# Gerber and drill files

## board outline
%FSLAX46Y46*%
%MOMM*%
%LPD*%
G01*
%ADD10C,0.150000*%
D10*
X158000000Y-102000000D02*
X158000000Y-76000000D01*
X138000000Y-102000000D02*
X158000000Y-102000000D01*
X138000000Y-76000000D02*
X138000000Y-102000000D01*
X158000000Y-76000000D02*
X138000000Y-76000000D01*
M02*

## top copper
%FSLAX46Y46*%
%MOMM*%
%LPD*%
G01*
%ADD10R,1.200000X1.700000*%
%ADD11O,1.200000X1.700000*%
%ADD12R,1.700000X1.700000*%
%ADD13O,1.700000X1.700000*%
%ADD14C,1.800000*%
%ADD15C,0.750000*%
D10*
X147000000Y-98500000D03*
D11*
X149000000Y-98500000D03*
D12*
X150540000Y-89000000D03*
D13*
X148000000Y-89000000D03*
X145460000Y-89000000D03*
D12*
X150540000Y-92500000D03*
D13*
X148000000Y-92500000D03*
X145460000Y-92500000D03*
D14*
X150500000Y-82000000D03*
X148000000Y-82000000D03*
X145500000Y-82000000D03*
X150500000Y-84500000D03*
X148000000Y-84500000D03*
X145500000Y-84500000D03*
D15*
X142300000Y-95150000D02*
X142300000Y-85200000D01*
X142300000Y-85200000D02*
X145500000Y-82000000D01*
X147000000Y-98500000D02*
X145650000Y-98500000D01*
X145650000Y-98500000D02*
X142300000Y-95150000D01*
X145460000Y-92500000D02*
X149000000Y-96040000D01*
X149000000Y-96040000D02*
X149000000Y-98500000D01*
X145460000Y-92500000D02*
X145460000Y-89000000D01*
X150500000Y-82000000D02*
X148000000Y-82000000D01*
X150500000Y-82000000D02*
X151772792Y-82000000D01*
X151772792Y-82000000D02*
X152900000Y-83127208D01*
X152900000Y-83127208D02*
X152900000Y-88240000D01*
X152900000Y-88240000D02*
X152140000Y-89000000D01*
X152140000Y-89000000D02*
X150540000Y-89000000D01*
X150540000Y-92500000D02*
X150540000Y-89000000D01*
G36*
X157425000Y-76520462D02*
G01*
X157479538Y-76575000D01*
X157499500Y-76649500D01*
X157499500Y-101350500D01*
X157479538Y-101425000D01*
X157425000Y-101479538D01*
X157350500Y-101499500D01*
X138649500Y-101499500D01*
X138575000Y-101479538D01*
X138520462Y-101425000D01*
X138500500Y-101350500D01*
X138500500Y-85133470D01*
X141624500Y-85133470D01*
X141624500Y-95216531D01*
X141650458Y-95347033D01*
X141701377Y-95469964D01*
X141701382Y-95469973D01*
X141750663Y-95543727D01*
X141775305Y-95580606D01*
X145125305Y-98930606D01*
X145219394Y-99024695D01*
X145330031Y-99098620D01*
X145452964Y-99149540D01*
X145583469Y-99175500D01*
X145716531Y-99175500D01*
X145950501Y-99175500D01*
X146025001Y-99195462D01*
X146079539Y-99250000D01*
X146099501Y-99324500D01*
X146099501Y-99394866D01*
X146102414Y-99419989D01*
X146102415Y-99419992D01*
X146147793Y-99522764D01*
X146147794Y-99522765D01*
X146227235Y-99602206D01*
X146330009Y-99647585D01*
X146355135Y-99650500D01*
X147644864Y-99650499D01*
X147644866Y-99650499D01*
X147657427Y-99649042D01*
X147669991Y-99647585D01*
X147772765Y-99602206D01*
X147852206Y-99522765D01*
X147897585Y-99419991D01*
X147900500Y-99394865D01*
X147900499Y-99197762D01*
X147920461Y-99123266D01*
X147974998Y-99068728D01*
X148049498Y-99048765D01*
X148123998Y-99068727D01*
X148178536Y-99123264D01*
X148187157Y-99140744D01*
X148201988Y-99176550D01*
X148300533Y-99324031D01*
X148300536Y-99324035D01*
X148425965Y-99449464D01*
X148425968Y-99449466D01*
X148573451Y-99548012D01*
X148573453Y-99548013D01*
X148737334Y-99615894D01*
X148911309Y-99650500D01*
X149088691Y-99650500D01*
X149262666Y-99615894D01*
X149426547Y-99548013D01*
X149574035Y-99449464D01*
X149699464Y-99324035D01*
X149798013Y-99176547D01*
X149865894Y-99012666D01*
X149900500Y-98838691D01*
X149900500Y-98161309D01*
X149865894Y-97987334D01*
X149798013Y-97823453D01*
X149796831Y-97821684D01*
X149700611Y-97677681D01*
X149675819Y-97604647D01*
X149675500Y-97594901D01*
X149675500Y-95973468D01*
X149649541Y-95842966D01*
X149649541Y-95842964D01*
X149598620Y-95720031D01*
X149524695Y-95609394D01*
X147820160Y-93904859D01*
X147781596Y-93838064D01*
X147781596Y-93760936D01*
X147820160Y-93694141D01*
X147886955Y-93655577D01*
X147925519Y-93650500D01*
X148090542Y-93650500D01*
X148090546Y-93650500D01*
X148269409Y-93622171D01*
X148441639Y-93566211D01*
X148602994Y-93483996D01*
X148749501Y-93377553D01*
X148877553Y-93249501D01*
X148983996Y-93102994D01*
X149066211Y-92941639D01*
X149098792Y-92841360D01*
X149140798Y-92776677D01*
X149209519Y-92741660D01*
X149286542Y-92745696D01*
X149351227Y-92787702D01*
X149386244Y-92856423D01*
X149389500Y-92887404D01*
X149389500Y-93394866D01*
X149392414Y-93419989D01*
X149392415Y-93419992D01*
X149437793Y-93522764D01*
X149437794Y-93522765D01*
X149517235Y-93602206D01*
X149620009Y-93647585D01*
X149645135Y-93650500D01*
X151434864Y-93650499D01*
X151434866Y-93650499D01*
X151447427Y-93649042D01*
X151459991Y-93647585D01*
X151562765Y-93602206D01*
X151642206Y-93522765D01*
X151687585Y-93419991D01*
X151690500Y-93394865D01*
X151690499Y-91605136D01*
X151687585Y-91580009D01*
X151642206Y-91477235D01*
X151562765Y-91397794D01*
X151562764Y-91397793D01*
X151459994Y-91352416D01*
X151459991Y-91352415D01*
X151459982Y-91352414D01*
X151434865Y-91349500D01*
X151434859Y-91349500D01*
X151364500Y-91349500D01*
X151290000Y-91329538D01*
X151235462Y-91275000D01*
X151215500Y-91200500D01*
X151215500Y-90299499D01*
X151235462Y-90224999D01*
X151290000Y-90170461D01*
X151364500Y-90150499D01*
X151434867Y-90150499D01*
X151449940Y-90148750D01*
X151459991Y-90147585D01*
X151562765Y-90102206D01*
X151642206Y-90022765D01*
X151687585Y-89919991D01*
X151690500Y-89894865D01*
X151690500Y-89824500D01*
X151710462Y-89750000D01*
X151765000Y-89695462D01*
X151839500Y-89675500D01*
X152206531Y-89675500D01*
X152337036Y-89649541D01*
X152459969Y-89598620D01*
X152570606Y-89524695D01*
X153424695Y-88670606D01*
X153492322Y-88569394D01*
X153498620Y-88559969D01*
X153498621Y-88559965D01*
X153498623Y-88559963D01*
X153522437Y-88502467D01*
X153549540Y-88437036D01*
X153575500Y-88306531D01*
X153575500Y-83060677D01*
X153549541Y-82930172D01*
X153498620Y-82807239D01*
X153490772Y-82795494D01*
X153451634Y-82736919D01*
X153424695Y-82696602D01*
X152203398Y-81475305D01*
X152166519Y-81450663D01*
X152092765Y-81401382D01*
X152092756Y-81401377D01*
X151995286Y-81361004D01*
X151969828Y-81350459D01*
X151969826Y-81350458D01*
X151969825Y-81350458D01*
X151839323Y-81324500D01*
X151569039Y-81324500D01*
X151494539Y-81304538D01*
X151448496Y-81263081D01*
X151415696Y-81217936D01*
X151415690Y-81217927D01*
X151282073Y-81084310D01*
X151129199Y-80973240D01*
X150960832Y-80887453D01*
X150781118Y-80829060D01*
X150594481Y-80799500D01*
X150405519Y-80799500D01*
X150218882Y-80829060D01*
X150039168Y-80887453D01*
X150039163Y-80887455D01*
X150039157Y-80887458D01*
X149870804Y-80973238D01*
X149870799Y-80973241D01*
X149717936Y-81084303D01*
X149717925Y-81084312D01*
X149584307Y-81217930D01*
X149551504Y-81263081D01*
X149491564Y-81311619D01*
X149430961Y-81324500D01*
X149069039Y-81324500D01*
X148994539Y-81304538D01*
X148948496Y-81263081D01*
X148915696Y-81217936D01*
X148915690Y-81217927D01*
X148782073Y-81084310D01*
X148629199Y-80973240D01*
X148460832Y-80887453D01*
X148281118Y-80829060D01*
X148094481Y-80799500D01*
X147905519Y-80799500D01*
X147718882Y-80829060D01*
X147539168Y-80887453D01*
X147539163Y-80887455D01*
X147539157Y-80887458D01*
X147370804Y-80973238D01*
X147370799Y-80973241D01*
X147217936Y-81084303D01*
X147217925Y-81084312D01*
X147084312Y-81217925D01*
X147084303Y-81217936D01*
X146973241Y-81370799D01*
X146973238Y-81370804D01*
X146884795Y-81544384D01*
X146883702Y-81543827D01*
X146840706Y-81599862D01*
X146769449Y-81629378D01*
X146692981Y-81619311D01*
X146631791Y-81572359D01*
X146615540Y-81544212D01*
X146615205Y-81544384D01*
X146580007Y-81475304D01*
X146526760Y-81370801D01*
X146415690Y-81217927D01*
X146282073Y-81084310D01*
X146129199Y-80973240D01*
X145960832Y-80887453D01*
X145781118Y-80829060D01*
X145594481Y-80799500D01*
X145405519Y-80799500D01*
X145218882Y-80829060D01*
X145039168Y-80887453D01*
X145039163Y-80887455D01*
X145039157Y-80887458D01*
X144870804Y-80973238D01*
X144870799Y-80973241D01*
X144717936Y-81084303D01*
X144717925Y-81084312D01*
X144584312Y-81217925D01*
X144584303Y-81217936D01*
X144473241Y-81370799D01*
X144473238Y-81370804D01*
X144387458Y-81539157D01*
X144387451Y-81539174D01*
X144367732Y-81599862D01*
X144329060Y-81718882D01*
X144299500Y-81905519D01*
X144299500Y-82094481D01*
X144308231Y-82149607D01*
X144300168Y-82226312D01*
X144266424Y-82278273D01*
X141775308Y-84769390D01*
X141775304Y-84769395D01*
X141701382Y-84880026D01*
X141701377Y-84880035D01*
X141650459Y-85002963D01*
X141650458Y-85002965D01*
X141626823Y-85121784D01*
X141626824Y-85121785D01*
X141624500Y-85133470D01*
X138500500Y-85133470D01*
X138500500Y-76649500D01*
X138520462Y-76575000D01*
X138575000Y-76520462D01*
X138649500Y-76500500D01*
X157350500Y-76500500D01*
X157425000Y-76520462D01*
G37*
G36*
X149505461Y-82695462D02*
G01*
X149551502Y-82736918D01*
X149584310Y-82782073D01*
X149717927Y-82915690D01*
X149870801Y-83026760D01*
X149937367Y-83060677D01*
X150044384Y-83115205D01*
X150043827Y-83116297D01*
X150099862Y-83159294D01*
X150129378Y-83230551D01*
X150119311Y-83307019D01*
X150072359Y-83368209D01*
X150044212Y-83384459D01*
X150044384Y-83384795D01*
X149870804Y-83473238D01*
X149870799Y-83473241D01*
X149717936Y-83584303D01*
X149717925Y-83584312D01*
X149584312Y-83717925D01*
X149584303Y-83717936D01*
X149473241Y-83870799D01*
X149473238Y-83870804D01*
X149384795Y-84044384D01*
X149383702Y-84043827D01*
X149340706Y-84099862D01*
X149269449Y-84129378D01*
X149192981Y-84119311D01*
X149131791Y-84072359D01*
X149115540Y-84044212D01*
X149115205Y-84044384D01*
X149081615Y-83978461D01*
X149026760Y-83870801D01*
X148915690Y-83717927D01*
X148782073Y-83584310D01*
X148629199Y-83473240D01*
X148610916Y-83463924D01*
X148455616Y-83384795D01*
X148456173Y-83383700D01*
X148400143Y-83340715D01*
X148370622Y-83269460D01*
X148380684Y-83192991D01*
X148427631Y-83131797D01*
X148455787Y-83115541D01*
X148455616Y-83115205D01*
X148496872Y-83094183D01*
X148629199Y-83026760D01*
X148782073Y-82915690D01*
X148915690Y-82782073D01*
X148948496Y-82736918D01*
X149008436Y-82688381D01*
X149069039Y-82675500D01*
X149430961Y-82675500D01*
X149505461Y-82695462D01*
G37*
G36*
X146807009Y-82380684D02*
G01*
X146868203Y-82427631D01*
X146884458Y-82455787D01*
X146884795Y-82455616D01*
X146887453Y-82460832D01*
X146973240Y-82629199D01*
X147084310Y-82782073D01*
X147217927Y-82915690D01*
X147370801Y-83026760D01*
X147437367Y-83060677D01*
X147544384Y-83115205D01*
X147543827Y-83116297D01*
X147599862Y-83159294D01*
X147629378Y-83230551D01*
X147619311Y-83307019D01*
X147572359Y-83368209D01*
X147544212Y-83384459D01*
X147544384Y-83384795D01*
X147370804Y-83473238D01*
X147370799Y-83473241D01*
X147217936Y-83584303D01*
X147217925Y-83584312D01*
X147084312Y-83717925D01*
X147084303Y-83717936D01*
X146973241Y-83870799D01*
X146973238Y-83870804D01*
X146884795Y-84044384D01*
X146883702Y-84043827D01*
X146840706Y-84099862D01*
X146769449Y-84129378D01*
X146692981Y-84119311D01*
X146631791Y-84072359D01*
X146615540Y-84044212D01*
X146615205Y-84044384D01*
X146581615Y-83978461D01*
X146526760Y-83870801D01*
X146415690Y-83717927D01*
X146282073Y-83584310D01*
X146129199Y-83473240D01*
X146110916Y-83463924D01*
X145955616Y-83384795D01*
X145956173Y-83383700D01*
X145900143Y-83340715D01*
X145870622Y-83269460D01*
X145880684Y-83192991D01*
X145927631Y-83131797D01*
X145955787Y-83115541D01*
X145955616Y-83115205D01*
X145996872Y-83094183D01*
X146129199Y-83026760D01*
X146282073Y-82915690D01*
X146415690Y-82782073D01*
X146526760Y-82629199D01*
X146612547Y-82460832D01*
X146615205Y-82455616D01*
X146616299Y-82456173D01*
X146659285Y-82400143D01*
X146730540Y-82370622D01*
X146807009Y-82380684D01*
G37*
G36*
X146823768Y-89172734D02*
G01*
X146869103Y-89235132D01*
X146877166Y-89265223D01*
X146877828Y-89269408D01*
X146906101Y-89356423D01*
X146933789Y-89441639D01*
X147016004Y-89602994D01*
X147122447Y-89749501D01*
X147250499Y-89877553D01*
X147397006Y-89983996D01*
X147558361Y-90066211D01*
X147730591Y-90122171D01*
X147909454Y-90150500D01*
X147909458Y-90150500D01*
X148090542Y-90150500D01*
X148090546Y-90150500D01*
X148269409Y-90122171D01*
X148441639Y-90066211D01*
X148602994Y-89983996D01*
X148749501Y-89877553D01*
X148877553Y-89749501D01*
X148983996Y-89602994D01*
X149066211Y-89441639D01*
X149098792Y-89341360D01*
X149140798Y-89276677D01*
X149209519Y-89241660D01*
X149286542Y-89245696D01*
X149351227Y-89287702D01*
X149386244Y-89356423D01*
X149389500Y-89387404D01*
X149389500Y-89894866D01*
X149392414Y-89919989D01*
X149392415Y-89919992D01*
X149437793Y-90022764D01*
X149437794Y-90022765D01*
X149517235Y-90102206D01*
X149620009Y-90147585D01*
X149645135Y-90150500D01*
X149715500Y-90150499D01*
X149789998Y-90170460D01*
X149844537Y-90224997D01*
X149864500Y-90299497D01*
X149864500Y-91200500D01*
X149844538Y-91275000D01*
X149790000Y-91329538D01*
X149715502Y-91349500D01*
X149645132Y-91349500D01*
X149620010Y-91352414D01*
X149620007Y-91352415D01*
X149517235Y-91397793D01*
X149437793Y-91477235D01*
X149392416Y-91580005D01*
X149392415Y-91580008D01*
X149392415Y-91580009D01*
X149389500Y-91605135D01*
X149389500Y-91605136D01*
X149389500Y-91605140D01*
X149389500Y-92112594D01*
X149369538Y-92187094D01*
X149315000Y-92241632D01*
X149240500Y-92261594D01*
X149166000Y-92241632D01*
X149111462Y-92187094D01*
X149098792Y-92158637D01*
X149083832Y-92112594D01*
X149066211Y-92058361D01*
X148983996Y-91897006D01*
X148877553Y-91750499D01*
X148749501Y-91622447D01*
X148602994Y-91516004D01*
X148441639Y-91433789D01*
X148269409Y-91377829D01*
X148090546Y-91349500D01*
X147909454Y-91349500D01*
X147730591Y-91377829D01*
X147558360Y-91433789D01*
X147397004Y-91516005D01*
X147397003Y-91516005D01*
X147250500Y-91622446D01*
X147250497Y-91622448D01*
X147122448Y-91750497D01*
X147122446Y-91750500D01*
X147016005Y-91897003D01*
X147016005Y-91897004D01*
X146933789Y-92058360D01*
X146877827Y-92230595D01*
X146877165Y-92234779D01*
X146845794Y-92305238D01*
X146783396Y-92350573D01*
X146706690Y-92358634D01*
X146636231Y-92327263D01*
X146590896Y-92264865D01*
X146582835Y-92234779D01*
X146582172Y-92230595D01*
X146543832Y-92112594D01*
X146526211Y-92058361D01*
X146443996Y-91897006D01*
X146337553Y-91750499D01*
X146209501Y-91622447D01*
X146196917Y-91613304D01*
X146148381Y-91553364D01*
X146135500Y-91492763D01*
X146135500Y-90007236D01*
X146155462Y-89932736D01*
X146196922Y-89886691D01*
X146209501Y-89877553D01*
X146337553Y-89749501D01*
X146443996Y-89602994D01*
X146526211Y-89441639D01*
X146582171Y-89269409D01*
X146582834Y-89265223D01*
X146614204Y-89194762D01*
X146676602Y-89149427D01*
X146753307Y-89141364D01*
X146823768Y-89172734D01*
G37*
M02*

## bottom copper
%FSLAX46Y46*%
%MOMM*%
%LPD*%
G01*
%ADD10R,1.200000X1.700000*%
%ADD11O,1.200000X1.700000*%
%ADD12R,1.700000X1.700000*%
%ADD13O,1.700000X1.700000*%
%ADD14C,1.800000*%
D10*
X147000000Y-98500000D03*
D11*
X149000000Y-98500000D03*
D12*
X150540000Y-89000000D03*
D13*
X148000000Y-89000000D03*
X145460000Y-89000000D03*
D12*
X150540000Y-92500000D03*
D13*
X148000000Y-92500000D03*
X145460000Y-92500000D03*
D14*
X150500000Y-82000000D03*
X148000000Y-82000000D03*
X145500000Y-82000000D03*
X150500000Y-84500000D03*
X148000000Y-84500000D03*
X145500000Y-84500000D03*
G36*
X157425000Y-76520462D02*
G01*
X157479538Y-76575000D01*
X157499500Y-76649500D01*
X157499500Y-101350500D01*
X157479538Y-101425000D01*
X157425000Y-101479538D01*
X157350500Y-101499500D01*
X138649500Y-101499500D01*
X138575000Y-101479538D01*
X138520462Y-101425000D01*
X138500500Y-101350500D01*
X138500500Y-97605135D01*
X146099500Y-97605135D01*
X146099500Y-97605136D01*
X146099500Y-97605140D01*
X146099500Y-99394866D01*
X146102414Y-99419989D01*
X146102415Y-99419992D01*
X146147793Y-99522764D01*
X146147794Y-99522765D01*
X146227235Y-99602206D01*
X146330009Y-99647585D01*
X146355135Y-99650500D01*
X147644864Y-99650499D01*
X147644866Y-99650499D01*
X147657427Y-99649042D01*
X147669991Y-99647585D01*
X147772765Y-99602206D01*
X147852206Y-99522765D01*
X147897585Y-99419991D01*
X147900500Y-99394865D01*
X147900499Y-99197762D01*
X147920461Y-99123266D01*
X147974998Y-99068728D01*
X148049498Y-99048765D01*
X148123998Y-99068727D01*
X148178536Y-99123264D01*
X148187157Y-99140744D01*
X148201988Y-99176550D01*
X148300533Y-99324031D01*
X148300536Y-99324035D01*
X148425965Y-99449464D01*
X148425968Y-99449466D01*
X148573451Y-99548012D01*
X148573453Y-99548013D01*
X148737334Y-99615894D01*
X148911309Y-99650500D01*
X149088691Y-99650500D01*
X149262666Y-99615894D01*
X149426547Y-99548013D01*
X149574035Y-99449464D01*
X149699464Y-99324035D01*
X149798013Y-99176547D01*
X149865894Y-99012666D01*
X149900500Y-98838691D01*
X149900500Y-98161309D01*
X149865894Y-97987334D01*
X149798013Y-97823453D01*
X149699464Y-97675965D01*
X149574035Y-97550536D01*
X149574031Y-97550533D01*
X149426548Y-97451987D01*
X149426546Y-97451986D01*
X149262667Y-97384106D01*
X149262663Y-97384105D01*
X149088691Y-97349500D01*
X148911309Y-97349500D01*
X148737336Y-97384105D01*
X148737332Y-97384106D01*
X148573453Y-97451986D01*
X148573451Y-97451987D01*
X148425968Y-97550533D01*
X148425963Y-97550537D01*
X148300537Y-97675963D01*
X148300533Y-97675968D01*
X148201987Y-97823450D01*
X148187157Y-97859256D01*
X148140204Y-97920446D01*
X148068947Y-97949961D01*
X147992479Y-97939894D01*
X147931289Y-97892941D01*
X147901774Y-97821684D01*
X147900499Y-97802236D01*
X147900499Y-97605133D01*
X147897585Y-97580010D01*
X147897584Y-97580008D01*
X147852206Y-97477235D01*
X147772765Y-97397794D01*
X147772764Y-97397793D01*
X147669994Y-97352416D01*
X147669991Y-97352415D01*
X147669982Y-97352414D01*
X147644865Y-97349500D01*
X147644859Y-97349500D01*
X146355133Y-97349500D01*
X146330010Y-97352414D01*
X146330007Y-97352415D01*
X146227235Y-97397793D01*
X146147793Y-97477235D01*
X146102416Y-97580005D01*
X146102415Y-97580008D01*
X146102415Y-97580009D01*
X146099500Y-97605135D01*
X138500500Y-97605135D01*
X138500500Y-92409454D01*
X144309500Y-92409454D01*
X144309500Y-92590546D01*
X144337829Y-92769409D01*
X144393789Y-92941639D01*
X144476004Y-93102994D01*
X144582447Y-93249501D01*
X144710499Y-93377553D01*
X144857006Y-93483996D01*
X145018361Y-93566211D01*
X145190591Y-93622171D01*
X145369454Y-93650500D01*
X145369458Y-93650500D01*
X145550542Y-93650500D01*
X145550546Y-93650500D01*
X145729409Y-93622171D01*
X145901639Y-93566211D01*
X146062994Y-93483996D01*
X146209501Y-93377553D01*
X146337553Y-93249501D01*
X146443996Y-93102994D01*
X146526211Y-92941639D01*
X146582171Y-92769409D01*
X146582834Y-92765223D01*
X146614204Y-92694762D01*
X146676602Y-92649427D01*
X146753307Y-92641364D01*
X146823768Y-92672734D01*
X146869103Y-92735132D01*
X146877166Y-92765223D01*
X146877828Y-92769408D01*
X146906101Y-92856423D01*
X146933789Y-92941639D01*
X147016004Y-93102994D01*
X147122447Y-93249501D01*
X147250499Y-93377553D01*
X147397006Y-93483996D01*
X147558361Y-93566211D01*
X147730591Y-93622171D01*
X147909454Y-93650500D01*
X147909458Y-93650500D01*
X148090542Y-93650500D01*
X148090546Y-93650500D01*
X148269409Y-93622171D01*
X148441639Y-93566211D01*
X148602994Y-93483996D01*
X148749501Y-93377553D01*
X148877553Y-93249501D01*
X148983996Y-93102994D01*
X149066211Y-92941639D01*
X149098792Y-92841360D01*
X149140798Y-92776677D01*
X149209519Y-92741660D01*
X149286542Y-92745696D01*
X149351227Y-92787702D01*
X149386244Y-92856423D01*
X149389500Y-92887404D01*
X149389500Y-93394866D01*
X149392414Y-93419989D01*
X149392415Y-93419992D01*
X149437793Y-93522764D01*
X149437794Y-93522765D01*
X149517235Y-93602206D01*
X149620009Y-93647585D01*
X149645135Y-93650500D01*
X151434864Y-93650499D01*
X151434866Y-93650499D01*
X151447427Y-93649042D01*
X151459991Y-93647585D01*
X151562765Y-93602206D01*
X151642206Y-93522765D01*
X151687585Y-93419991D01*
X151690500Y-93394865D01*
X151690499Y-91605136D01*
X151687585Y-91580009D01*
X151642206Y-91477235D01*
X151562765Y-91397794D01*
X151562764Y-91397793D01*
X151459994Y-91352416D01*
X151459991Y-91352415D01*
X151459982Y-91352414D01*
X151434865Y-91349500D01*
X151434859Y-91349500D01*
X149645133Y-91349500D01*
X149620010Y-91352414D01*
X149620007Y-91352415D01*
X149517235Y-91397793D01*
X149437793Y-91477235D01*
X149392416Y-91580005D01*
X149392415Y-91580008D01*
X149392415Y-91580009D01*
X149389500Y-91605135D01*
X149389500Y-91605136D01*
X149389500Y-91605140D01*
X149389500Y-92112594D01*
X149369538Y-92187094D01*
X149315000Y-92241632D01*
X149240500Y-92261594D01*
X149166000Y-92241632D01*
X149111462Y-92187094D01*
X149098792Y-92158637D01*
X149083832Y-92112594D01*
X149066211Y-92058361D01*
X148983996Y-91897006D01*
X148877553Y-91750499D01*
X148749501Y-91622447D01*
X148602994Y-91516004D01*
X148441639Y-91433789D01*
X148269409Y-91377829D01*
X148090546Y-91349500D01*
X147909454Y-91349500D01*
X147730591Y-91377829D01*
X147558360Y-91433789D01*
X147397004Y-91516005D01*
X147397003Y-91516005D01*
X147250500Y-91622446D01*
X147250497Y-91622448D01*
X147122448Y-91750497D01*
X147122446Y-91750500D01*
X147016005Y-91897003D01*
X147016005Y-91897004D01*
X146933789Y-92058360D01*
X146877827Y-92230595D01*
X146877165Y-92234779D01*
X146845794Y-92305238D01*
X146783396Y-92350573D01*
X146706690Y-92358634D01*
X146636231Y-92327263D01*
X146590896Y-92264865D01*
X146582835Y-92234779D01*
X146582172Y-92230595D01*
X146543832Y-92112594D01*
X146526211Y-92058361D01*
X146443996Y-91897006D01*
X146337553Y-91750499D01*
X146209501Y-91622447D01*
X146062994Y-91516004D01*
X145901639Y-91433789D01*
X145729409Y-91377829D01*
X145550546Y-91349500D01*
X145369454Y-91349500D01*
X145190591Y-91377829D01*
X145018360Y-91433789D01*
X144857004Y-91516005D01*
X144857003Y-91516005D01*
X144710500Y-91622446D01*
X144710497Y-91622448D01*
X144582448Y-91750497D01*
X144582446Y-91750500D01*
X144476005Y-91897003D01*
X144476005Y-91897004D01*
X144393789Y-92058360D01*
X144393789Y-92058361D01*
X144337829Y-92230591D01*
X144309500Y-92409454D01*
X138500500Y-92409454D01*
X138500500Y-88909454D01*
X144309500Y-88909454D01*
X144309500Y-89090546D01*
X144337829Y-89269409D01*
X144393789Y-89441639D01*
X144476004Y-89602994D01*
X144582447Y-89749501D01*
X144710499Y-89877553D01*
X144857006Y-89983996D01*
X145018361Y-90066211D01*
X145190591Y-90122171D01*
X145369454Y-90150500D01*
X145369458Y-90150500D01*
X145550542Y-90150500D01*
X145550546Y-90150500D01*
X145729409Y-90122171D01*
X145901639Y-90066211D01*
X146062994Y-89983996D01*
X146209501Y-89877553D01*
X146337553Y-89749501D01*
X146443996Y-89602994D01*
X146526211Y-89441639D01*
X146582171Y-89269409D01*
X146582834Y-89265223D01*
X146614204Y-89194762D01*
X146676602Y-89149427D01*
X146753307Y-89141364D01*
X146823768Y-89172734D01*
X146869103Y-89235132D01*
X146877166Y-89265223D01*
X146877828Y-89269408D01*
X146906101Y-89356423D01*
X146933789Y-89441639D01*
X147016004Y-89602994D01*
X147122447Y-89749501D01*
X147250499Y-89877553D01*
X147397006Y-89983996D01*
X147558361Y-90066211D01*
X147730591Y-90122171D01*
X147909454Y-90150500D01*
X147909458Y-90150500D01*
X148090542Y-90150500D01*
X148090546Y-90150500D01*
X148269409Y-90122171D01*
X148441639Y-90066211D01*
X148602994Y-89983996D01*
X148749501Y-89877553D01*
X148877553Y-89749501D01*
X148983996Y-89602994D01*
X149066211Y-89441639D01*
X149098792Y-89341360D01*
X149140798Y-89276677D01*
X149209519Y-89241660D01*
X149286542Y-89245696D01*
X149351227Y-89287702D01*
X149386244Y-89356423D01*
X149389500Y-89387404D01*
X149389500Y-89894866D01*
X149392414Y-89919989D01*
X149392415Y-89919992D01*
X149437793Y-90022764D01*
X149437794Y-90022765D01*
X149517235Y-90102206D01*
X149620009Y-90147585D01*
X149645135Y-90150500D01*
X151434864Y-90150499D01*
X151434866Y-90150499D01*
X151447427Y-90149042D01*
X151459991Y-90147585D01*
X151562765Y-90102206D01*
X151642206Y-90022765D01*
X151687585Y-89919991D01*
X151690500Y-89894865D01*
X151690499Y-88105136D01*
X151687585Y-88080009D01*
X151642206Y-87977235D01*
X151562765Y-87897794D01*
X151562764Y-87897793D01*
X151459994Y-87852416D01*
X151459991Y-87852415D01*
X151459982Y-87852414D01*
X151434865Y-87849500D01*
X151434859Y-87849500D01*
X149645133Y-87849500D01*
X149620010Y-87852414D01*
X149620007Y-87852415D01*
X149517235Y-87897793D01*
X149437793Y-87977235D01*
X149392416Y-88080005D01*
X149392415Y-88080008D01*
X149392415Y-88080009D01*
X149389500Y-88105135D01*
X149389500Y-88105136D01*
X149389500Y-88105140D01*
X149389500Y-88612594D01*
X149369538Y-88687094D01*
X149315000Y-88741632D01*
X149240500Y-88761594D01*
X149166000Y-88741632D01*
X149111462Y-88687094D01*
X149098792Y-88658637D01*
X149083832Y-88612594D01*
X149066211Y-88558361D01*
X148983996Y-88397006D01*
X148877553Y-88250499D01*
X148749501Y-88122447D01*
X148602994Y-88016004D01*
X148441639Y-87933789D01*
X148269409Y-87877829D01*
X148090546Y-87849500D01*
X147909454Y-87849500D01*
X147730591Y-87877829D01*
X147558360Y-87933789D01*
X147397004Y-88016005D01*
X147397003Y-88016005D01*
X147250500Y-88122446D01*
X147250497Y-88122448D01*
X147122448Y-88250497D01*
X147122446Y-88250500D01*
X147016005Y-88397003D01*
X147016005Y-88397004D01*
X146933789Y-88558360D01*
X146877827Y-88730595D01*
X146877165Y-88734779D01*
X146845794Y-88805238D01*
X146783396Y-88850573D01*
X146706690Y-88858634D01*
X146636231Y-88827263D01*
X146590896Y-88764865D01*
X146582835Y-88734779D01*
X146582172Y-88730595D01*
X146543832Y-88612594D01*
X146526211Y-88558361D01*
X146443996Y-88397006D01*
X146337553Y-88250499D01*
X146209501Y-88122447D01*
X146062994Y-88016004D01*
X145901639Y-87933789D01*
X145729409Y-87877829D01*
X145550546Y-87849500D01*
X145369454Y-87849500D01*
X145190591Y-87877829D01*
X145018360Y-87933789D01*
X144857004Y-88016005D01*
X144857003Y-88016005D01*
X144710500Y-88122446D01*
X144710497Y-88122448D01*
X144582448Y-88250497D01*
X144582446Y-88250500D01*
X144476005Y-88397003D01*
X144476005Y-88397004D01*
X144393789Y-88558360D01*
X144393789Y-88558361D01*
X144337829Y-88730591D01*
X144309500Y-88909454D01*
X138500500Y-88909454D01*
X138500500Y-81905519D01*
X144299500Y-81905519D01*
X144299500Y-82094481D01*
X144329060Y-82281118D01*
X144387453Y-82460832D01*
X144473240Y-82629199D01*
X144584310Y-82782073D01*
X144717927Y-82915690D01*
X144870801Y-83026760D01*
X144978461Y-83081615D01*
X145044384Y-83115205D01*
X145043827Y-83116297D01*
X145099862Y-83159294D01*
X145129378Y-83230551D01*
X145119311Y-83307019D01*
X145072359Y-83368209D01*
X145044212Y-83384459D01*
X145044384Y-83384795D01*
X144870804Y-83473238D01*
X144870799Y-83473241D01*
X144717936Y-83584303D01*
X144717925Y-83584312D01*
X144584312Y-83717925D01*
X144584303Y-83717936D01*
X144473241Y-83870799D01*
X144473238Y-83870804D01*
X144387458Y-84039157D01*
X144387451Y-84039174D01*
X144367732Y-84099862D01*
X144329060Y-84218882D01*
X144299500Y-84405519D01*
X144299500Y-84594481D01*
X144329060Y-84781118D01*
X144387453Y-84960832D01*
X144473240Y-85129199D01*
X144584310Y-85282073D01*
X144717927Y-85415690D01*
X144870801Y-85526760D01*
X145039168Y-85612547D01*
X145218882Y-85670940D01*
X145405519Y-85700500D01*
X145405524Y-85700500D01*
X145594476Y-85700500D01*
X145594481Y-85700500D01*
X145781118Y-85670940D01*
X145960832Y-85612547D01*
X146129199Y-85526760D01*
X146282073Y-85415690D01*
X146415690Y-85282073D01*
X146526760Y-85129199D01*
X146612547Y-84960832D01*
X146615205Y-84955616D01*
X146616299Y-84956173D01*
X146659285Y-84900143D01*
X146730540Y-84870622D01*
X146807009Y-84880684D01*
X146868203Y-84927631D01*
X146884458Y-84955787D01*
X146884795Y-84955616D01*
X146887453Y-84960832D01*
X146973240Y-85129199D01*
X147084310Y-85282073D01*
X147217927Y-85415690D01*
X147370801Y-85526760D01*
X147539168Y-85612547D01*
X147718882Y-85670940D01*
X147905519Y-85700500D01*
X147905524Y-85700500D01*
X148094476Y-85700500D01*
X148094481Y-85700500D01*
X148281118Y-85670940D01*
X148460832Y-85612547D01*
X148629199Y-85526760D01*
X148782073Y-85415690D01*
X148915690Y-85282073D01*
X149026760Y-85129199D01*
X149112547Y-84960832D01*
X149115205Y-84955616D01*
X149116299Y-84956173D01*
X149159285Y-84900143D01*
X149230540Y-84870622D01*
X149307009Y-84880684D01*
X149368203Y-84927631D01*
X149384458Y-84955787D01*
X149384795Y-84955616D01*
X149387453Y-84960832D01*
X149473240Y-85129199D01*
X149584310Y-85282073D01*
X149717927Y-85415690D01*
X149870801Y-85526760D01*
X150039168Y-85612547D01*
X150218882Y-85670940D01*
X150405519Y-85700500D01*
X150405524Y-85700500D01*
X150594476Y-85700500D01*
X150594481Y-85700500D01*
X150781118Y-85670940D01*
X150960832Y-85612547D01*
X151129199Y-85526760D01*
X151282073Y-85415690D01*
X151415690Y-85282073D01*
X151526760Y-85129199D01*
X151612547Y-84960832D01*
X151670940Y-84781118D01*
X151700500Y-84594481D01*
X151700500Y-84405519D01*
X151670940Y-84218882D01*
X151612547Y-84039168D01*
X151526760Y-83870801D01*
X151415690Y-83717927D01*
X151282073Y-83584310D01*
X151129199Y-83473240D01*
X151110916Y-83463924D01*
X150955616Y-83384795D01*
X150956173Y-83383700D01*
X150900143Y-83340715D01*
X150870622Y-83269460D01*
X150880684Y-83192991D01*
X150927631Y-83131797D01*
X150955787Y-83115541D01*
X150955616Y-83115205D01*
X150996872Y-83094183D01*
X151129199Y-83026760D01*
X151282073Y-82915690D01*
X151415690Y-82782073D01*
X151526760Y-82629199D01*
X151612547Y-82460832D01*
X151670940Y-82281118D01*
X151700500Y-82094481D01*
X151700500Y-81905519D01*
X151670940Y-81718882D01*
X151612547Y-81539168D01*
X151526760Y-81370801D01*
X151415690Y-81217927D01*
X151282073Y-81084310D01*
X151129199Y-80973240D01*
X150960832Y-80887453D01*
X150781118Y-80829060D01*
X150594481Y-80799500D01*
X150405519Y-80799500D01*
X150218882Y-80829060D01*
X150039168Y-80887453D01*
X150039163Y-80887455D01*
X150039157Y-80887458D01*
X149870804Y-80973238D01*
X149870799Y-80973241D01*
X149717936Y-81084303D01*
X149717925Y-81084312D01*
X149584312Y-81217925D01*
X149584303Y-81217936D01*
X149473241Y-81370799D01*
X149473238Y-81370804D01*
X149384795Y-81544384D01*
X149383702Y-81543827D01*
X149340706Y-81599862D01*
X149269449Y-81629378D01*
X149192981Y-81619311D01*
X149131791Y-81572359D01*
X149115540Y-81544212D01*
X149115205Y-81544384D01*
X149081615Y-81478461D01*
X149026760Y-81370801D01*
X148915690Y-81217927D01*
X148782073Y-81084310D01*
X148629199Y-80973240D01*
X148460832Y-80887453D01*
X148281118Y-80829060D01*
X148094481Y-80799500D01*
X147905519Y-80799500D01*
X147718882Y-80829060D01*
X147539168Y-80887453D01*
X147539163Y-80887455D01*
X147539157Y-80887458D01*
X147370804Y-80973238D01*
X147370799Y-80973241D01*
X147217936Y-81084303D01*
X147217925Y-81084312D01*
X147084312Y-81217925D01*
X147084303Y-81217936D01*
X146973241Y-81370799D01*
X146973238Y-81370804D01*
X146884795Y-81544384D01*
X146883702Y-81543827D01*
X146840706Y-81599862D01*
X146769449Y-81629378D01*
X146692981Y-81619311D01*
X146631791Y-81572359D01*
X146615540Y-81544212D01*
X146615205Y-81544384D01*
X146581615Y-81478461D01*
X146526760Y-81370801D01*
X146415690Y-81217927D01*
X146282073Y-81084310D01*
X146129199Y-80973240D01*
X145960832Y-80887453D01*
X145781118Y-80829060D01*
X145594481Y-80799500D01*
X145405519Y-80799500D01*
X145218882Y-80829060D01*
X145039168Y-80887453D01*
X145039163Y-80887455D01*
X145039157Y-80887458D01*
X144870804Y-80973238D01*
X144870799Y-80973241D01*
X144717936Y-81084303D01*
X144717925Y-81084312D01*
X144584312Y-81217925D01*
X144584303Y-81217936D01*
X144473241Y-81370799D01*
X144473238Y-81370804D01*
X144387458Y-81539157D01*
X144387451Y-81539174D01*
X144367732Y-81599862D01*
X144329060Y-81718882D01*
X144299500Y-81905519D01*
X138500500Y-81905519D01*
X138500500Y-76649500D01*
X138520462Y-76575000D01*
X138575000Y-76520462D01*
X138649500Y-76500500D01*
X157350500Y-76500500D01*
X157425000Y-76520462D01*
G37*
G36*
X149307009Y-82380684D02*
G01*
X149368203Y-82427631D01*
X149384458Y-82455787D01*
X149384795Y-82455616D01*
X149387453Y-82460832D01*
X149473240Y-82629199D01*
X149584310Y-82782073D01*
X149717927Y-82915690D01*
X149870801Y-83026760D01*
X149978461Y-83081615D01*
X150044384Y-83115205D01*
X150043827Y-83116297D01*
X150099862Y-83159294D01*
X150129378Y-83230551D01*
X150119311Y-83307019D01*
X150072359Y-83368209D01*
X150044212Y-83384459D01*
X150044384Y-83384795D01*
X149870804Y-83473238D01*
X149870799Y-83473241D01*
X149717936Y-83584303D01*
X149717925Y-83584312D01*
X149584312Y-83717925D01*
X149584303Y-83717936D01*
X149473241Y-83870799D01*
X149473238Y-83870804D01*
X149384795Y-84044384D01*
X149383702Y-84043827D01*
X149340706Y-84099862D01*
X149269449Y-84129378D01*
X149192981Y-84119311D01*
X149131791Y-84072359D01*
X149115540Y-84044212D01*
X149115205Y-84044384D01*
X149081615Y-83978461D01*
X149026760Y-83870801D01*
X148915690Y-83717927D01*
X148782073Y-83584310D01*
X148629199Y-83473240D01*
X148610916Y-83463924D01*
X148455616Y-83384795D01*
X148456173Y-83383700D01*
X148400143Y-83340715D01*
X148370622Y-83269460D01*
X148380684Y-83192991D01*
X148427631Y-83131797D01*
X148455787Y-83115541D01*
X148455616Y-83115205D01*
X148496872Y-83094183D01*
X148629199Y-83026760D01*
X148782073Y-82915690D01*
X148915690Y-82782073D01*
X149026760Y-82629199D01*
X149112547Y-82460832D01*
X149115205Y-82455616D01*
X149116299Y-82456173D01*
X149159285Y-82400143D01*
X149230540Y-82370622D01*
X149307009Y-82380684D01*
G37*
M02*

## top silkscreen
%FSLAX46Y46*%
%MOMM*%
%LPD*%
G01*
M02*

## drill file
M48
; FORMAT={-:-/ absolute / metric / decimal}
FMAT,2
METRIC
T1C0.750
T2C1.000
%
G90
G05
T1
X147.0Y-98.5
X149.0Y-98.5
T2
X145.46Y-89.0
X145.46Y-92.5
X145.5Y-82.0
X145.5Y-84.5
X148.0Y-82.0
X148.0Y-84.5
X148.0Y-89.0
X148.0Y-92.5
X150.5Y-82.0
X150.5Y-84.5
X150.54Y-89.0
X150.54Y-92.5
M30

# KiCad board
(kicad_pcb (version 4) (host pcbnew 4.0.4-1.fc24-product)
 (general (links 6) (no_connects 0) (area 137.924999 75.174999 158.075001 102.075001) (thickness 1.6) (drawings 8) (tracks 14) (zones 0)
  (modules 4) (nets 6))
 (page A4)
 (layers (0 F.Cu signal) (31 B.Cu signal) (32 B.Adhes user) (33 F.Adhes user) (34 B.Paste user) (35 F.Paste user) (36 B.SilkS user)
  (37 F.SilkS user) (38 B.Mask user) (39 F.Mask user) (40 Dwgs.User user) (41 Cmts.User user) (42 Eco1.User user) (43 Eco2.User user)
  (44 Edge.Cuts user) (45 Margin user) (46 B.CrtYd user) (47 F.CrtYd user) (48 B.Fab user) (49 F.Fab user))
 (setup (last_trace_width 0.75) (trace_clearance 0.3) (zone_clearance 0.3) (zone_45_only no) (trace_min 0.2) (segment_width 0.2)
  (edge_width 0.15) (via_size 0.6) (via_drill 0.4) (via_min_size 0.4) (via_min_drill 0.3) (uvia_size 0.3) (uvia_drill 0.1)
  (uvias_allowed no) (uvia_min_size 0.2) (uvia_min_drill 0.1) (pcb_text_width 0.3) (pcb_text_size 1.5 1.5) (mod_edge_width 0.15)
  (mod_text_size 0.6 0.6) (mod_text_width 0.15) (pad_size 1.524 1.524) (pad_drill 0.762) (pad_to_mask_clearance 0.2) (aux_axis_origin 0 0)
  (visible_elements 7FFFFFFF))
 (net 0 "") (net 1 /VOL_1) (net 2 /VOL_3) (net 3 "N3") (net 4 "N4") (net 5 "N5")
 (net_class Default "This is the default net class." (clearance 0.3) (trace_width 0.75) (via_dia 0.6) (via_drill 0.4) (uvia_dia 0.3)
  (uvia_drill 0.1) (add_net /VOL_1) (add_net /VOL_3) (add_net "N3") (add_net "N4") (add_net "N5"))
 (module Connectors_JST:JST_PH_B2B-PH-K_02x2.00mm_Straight (layer B.Cu) (at 147 98.5)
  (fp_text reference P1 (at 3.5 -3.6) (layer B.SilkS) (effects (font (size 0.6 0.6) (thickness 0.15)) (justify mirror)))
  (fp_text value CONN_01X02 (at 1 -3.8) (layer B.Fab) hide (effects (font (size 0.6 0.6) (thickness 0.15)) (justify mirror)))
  (pad 1 thru_hole rect (at 0 0) (size 1.2 1.7) (drill 0.75) (layers *.Cu *.Mask) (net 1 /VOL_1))
  (pad 2 thru_hole oval (at 2 0) (size 1.2 1.7) (drill 0.75) (layers *.Cu *.Mask) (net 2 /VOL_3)))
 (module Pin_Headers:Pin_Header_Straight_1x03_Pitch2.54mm (layer B.Cu) (at 150.54 89 90)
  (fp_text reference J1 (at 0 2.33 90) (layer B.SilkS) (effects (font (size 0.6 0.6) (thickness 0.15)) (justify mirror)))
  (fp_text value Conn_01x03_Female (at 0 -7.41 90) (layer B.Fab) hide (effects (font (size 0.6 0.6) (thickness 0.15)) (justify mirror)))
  (pad 1 thru_hole rect (at 0 0 90) (size 1.7 1.7) (drill 1) (layers *.Cu *.Mask) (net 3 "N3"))
  (pad 2 thru_hole oval (at 0 -2.54 90) (size 1.7 1.7) (drill 1) (layers *.Cu *.Mask) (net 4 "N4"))
  (pad 3 thru_hole oval (at 0 -5.08 90) (size 1.7 1.7) (drill 1) (layers *.Cu *.Mask) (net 2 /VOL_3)))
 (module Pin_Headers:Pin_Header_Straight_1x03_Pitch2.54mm (layer B.Cu) (at 150.54 92.5 90)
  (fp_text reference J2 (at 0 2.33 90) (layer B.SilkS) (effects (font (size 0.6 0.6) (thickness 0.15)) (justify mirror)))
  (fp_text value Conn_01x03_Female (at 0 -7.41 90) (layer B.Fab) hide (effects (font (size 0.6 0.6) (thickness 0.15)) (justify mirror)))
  (pad 1 thru_hole rect (at 0 0 90) (size 1.7 1.7) (drill 1) (layers *.Cu *.Mask) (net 3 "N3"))
  (pad 2 thru_hole oval (at 0 -2.54 90) (size 1.7 1.7) (drill 1) (layers *.Cu *.Mask) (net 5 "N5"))
  (pad 3 thru_hole oval (at 0 -5.08 90) (size 1.7 1.7) (drill 1) (layers *.Cu *.Mask) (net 2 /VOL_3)))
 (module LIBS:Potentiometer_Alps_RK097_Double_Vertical (layer B.Cu) (at 145.5 82 90)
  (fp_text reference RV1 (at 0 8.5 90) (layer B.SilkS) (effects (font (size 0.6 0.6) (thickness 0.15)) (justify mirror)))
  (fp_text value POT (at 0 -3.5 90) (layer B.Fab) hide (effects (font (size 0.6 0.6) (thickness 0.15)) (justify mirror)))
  (pad 3 thru_hole circle (at 0 5 90) (size 1.8 1.8) (drill 1) (layers *.Cu *.Mask) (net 3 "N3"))
  (pad 2 thru_hole circle (at 0 2.5 90) (size 1.8 1.8) (drill 1) (layers *.Cu *.Mask) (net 3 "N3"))
  (pad 1 thru_hole circle (at 0 0 90) (size 1.8 1.8) (drill 1) (layers *.Cu *.Mask) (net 1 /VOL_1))
  (pad 6 thru_hole circle (at -2.5 5 90) (size 1.8 1.8) (drill 1) (layers *.Cu *.Mask))
  (pad 5 thru_hole circle (at -2.5 2.5 90) (size 1.8 1.8) (drill 1) (layers *.Cu *.Mask))
  (pad 4 thru_hole circle (at -2.5 0 90) (size 1.8 1.8) (drill 1) (layers *.Cu *.Mask)))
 (gr_line (start 158 102) (end 158 76) (layer Edge.Cuts) (width 0.15))
 (gr_line (start 138 102) (end 158 102) (layer Edge.Cuts) (width 0.15))
 (gr_line (start 138 76) (end 138 102) (layer Edge.Cuts) (width 0.15))
 (gr_line (start 158 76) (end 138 76) (layer Edge.Cuts) (width 0.15))
 (segment (start 142.3 95.15) (end 142.3 85.2) (width 0.75) (layer F.Cu) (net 1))
 (segment (start 142.3 85.2) (end 145.5 82) (width 0.75) (layer F.Cu) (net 1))
 (segment (start 147 98.5) (end 145.65 98.5) (width 0.75) (layer F.Cu) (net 1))
 (segment (start 145.65 98.5) (end 142.3 95.15) (width 0.75) (layer F.Cu) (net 1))
 (segment (start 145.46 92.5) (end 149 96.04) (width 0.75) (layer F.Cu) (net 2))
 (segment (start 149 96.04) (end 149 98.5) (width 0.75) (layer F.Cu) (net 2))
 (segment (start 145.46 92.5) (end 145.46 89) (width 0.75) (layer F.Cu) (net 2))
 (segment (start 150.5 82) (end 148 82) (width 0.75) (layer F.Cu) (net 3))
 (segment (start 150.5 82) (end 151.772792 82) (width 0.75) (layer F.Cu) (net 3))
 (segment (start 151.772792 82) (end 152.9 83.127208) (width 0.75) (layer F.Cu) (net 3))
 (segment (start 152.9 83.127208) (end 152.9 88.24) (width 0.75) (layer F.Cu) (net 3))
 (segment (start 152.9 88.24) (end 152.14 89) (width 0.75) (layer F.Cu) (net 3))
 (segment (start 152.14 89) (end 150.54 89) (width 0.75) (layer F.Cu) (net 3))
 (segment (start 150.54 92.5) (end 150.54 89) (width 0.75) (layer F.Cu) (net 3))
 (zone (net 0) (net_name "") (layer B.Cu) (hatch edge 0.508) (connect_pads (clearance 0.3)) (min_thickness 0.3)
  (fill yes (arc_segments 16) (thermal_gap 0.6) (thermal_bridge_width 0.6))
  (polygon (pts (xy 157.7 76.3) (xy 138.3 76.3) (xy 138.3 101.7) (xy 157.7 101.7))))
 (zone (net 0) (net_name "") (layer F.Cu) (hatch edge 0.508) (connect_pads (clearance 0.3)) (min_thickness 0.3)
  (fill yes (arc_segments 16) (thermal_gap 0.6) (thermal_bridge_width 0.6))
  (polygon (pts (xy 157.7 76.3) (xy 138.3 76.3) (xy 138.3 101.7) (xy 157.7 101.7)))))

